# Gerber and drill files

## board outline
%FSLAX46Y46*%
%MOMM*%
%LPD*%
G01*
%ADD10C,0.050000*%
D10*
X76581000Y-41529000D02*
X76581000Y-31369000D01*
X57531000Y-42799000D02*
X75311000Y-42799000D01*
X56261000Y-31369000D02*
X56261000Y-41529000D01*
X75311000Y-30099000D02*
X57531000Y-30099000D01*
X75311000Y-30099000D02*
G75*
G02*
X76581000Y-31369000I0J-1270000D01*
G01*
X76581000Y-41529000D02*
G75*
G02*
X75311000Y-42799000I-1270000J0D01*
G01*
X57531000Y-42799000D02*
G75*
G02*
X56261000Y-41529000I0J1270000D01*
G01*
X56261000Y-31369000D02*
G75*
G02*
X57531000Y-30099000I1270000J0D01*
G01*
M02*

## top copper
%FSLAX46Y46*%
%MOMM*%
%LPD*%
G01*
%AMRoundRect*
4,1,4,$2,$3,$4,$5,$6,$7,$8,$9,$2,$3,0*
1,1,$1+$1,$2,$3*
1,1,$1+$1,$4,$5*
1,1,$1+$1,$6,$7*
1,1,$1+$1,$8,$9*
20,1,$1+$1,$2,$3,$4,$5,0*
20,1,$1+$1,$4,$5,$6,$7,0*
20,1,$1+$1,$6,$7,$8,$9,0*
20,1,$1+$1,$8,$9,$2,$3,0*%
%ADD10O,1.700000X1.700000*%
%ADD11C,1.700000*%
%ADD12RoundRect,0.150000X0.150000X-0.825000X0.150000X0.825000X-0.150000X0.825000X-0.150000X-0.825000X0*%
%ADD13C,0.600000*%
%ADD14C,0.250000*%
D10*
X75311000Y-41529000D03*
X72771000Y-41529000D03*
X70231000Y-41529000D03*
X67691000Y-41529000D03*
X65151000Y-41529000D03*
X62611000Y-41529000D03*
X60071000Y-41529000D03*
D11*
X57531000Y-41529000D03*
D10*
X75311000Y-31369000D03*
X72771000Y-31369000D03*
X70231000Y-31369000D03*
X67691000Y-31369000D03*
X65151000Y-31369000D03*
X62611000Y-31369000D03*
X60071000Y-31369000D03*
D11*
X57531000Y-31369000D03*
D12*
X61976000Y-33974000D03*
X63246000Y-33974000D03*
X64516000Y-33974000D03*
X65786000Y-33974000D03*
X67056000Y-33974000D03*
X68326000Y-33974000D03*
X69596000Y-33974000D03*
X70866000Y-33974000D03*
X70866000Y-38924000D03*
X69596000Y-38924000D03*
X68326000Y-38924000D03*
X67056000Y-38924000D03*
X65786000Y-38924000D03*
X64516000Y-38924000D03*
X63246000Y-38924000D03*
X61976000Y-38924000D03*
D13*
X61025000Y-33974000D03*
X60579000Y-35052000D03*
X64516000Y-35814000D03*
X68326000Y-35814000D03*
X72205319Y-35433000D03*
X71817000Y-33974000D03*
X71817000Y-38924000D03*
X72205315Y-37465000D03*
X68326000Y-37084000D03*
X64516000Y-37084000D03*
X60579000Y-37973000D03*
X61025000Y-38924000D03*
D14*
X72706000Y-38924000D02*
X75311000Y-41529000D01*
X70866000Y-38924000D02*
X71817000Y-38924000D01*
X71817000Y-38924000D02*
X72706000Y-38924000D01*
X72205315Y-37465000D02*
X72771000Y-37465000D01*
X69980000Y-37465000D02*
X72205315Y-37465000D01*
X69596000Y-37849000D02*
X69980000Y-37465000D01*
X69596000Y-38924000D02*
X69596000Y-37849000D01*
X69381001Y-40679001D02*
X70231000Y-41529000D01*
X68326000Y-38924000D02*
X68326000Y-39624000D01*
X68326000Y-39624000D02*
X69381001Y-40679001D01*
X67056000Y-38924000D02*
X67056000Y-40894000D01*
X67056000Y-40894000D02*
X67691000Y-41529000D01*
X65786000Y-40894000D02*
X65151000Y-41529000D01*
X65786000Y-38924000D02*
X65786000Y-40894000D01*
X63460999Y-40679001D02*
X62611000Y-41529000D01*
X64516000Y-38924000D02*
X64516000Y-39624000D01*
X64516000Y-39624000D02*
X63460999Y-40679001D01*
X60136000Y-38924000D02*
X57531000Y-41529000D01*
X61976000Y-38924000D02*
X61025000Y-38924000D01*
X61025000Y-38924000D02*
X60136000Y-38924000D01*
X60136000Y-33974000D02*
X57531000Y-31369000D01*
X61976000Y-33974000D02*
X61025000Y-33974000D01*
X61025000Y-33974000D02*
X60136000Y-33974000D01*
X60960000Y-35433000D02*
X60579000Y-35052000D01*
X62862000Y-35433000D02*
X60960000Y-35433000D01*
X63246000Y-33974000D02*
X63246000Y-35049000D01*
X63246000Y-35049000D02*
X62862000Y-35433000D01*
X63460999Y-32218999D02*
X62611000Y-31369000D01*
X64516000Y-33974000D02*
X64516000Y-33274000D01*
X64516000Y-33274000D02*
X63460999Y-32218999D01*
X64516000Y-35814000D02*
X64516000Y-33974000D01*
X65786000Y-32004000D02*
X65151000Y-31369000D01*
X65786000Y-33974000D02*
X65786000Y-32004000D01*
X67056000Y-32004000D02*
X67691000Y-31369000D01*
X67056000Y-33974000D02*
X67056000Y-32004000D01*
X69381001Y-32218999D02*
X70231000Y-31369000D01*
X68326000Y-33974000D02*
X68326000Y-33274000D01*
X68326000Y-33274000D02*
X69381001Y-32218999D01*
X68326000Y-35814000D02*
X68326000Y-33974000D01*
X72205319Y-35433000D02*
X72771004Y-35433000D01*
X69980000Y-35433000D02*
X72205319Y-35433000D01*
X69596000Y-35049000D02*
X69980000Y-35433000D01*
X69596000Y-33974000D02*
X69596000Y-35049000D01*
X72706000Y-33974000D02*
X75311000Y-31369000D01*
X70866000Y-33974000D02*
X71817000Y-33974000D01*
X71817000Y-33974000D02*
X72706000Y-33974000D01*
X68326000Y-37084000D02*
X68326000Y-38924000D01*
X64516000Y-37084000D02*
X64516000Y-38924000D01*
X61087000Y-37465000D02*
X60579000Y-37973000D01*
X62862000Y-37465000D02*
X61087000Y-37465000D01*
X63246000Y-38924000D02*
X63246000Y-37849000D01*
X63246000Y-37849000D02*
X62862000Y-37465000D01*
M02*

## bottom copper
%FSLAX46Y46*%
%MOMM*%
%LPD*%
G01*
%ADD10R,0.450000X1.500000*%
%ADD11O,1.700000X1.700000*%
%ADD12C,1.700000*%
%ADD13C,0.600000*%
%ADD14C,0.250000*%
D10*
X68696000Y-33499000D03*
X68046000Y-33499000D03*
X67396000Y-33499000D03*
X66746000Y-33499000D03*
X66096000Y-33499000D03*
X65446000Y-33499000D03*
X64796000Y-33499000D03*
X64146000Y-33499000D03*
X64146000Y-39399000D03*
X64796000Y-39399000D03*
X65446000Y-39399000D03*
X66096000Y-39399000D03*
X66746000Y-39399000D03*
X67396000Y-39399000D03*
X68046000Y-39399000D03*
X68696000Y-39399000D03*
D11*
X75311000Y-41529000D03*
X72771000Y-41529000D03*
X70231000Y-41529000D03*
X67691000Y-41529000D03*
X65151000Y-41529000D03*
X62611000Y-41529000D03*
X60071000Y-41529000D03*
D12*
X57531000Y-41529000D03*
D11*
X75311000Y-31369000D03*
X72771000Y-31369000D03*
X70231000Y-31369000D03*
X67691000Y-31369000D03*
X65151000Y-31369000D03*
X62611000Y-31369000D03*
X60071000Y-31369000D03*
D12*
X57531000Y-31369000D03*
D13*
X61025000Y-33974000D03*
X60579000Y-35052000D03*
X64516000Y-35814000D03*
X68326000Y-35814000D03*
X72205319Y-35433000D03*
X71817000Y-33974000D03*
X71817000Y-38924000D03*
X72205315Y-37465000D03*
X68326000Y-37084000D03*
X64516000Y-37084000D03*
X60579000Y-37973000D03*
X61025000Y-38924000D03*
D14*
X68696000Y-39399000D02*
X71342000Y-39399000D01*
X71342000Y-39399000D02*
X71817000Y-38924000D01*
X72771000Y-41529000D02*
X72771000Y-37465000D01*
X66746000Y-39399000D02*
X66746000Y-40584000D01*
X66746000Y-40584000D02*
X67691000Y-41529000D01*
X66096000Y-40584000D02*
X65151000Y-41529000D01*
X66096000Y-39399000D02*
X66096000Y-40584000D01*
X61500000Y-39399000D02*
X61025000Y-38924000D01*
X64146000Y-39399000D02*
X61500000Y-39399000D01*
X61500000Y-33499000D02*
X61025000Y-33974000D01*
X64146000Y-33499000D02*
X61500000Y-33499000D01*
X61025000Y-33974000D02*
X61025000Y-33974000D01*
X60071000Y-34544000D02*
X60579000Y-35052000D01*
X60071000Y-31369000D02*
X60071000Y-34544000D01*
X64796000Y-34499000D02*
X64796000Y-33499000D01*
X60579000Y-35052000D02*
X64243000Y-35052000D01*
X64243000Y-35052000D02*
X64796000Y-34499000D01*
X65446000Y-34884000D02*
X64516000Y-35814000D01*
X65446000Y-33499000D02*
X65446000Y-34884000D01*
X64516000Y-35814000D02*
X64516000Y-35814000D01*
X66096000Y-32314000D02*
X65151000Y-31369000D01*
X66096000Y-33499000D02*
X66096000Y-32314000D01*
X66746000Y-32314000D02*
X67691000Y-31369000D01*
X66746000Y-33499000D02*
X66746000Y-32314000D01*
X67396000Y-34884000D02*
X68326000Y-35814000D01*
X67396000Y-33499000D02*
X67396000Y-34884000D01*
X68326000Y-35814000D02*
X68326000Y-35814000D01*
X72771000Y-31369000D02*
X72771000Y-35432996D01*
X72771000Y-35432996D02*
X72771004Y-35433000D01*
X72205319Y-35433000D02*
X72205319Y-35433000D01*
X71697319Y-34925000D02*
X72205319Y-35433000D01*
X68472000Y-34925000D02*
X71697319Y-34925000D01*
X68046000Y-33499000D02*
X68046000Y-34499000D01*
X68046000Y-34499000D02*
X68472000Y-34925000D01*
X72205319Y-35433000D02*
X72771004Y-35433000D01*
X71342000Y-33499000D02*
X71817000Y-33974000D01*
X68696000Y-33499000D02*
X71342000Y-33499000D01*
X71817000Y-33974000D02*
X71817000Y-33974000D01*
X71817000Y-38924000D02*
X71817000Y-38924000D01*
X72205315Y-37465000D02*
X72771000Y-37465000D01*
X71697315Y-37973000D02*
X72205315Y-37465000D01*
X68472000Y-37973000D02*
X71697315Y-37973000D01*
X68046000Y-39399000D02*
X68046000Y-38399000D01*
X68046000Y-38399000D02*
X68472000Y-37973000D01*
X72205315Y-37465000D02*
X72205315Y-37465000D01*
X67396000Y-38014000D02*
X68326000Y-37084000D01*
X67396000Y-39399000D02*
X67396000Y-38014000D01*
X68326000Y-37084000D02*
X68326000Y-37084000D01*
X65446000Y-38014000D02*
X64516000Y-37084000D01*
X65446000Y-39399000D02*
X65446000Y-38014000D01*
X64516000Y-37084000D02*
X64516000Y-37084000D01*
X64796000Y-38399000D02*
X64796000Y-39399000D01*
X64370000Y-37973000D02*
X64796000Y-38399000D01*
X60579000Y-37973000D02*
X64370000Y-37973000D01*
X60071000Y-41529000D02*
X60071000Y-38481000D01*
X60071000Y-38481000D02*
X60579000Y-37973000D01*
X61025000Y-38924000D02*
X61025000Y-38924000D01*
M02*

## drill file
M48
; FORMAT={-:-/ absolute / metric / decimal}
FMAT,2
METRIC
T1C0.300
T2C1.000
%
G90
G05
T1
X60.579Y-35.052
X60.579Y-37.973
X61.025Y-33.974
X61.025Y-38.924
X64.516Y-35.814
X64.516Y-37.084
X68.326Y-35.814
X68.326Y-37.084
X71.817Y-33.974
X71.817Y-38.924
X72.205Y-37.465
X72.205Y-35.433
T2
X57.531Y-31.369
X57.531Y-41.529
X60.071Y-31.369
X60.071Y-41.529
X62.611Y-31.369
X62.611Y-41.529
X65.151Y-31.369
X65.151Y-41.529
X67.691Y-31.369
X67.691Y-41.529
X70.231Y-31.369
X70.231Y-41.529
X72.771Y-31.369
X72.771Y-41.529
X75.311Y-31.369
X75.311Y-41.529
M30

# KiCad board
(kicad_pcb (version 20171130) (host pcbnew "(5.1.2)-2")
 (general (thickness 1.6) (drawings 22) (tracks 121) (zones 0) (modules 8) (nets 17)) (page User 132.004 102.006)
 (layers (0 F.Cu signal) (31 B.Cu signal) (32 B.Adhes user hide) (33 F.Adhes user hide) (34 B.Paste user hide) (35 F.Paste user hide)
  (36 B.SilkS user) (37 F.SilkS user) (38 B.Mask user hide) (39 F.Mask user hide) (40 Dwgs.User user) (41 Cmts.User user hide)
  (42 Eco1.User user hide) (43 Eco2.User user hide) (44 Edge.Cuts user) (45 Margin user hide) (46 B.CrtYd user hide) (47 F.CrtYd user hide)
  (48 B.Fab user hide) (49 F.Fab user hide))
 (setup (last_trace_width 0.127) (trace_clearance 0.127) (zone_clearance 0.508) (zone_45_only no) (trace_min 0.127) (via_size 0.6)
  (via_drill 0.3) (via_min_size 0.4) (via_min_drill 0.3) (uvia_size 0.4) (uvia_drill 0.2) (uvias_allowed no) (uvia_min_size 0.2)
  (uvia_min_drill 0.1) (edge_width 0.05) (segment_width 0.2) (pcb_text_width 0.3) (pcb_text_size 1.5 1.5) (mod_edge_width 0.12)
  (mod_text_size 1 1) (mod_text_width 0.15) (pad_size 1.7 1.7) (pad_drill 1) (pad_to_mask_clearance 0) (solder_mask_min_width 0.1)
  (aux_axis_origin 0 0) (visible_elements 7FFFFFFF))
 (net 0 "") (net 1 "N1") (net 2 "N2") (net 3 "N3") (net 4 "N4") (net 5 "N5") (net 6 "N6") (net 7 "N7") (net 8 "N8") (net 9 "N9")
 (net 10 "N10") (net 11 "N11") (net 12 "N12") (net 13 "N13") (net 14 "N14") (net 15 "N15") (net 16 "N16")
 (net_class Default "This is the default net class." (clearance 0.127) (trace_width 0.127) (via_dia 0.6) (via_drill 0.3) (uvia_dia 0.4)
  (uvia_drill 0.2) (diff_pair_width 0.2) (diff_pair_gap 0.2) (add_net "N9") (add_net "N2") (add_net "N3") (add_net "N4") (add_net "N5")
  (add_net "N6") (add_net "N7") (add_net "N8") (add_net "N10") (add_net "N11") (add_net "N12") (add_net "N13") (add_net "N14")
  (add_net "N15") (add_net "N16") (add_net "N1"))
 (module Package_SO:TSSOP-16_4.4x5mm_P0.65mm (layer B.Cu) (at 66.421 36.449 90)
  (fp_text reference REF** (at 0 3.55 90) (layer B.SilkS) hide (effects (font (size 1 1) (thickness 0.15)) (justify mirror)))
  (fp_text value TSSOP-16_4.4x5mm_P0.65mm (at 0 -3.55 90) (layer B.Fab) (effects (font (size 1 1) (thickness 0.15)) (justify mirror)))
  (pad 16 smd rect (at 2.95 2.275 90) (size 1.5 0.45) (layers B.Cu B.Paste B.Mask) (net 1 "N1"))
  (pad 15 smd rect (at 2.95 1.625 90) (size 1.5 0.45) (layers B.Cu B.Paste B.Mask) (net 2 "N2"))
  (pad 14 smd rect (at 2.95 0.975 90) (size 1.5 0.45) (layers B.Cu B.Paste B.Mask) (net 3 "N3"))
  (pad 13 smd rect (at 2.95 0.325 90) (size 1.5 0.45) (layers B.Cu B.Paste B.Mask) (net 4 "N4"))
  (pad 12 smd rect (at 2.95 -0.325 90) (size 1.5 0.45) (layers B.Cu B.Paste B.Mask) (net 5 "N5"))
  (pad 11 smd rect (at 2.95 -0.975 90) (size 1.5 0.45) (layers B.Cu B.Paste B.Mask) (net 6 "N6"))
  (pad 10 smd rect (at 2.95 -1.625 90) (size 1.5 0.45) (layers B.Cu B.Paste B.Mask) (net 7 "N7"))
  (pad 9 smd rect (at 2.95 -2.275 90) (size 1.5 0.45) (layers B.Cu B.Paste B.Mask) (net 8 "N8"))
  (pad 8 smd rect (at -2.95 -2.275 90) (size 1.5 0.45) (layers B.Cu B.Paste B.Mask) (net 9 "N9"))
  (pad 7 smd rect (at -2.95 -1.625 90) (size 1.5 0.45) (layers B.Cu B.Paste B.Mask) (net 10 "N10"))
  (pad 6 smd rect (at -2.95 -0.975 90) (size 1.5 0.45) (layers B.Cu B.Paste B.Mask) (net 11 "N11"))
  (pad 5 smd rect (at -2.95 -0.325 90) (size 1.5 0.45) (layers B.Cu B.Paste B.Mask) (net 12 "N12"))
  (pad 4 smd rect (at -2.95 0.325 90) (size 1.5 0.45) (layers B.Cu B.Paste B.Mask) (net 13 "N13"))
  (pad 3 smd rect (at -2.95 0.975 90) (size 1.5 0.45) (layers B.Cu B.Paste B.Mask) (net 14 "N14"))
  (pad 2 smd rect (at -2.95 1.625 90) (size 1.5 0.45) (layers B.Cu B.Paste B.Mask) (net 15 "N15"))
  (pad 1 smd rect (at -2.95 2.275 90) (size 1.5 0.45) (layers B.Cu B.Paste B.Mask) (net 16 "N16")))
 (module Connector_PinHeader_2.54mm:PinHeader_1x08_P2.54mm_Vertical (layer F.Cu) (at 57.531 41.529 90)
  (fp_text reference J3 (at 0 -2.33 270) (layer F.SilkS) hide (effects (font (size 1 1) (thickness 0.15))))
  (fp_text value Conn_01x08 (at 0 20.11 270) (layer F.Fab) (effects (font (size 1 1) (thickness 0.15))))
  (pad 8 thru_hole oval (at 0 17.78 90) (size 1.7 1.7) (drill 1) (layers *.Cu *.Mask) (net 16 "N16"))
  (pad 7 thru_hole oval (at 0 15.24 90) (size 1.7 1.7) (drill 1) (layers *.Cu *.Mask) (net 15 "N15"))
  (pad 6 thru_hole oval (at 0 12.7 90) (size 1.7 1.7) (drill 1) (layers *.Cu *.Mask) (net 14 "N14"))
  (pad 5 thru_hole oval (at 0 10.16 90) (size 1.7 1.7) (drill 1) (layers *.Cu *.Mask) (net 13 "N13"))
  (pad 4 thru_hole oval (at 0 7.62 90) (size 1.7 1.7) (drill 1) (layers *.Cu *.Mask) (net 12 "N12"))
  (pad 3 thru_hole oval (at 0 5.08 90) (size 1.7 1.7) (drill 1) (layers *.Cu *.Mask) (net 11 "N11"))
  (pad 2 thru_hole oval (at 0 2.54 90) (size 1.7 1.7) (drill 1) (layers *.Cu *.Mask) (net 10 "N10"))
  (pad 1 thru_hole circle (at 0 0 90) (size 1.7 1.7) (drill 1) (layers *.Cu *.Mask) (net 9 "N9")))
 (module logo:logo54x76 (layer F.Cu) (at 58.801 36.703)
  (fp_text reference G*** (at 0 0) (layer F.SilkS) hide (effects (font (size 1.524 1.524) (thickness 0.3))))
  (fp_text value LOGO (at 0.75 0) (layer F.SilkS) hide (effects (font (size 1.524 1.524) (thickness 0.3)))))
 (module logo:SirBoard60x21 (layer F.Cu) (at 66.421 36.449)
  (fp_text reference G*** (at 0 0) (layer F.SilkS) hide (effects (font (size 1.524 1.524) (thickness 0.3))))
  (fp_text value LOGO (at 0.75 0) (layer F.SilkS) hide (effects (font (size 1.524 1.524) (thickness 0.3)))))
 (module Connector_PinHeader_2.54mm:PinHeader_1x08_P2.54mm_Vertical (layer F.Cu) (at 57.531 31.369 90)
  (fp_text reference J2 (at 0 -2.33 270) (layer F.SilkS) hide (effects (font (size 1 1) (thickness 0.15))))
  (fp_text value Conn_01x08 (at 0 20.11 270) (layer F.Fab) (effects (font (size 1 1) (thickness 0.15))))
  (pad 8 thru_hole oval (at 0 17.78 90) (size 1.7 1.7) (drill 1) (layers *.Cu *.Mask) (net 1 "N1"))
  (pad 7 thru_hole oval (at 0 15.24 90) (size 1.7 1.7) (drill 1) (layers *.Cu *.Mask) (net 2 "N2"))
  (pad 6 thru_hole oval (at 0 12.7 90) (size 1.7 1.7) (drill 1) (layers *.Cu *.Mask) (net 3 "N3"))
  (pad 5 thru_hole oval (at 0 10.16 90) (size 1.7 1.7) (drill 1) (layers *.Cu *.Mask) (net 4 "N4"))
  (pad 4 thru_hole oval (at 0 7.62 90) (size 1.7 1.7) (drill 1) (layers *.Cu *.Mask) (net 5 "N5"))
  (pad 3 thru_hole oval (at 0 5.08 90) (size 1.7 1.7) (drill 1) (layers *.Cu *.Mask) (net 6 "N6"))
  (pad 2 thru_hole oval (at 0 2.54 90) (size 1.7 1.7) (drill 1) (layers *.Cu *.Mask) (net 7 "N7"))
  (pad 1 thru_hole circle (at 0 0 90) (size 1.7 1.7) (drill 1) (layers *.Cu *.Mask) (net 8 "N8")))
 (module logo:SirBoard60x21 (layer B.Cu) (at 59.182 36.449 90)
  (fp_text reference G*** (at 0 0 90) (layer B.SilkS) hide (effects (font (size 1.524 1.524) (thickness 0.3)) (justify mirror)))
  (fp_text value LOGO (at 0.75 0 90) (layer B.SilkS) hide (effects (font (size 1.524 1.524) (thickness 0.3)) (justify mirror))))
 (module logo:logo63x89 (layer B.Cu) (at 73.025 36.576 90)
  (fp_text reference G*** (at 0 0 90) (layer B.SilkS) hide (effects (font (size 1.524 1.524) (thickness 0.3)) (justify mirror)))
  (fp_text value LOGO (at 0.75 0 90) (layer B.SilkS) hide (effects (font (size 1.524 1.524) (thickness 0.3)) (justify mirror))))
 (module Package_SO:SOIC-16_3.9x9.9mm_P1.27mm (layer F.Cu) (at 66.421 36.449 90)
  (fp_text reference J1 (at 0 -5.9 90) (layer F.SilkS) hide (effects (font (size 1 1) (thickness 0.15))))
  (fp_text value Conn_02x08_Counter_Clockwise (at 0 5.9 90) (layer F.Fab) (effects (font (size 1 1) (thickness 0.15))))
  (pad 16 smd roundrect (at 2.475 -4.445 90) (size 1.95 0.6) (layers F.Cu F.Paste F.Mask) (roundrect_rratio 0.25) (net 8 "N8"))
  (pad 15 smd roundrect (at 2.475 -3.175 90) (size 1.95 0.6) (layers F.Cu F.Paste F.Mask) (roundrect_rratio 0.25) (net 7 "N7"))
  (pad 14 smd roundrect (at 2.475 -1.905 90) (size 1.95 0.6) (layers F.Cu F.Paste F.Mask) (roundrect_rratio 0.25) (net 6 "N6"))
  (pad 13 smd roundrect (at 2.475 -0.635 90) (size 1.95 0.6) (layers F.Cu F.Paste F.Mask) (roundrect_rratio 0.25) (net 5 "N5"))
  (pad 12 smd roundrect (at 2.475 0.635 90) (size 1.95 0.6) (layers F.Cu F.Paste F.Mask) (roundrect_rratio 0.25) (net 4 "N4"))
  (pad 11 smd roundrect (at 2.475 1.905 90) (size 1.95 0.6) (layers F.Cu F.Paste F.Mask) (roundrect_rratio 0.25) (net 3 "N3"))
  (pad 10 smd roundrect (at 2.475 3.175 90) (size 1.95 0.6) (layers F.Cu F.Paste F.Mask) (roundrect_rratio 0.25) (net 2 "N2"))
  (pad 9 smd roundrect (at 2.475 4.445 90) (size 1.95 0.6) (layers F.Cu F.Paste F.Mask) (roundrect_rratio 0.25) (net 1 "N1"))
  (pad 8 smd roundrect (at -2.475 4.445 90) (size 1.95 0.6) (layers F.Cu F.Paste F.Mask) (roundrect_rratio 0.25) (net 16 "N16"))
  (pad 7 smd roundrect (at -2.475 3.175 90) (size 1.95 0.6) (layers F.Cu F.Paste F.Mask) (roundrect_rratio 0.25) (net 15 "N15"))
  (pad 6 smd roundrect (at -2.475 1.905 90) (size 1.95 0.6) (layers F.Cu F.Paste F.Mask) (roundrect_rratio 0.25) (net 14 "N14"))
  (pad 5 smd roundrect (at -2.475 0.635 90) (size 1.95 0.6) (layers F.Cu F.Paste F.Mask) (roundrect_rratio 0.25) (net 13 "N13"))
  (pad 4 smd roundrect (at -2.475 -0.635 90) (size 1.95 0.6) (layers F.Cu F.Paste F.Mask) (roundrect_rratio 0.25) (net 12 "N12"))
  (pad 3 smd roundrect (at -2.475 -1.905 90) (size 1.95 0.6) (layers F.Cu F.Paste F.Mask) (roundrect_rratio 0.25) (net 11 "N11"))
  (pad 2 smd roundrect (at -2.475 -3.175 90) (size 1.95 0.6) (layers F.Cu F.Paste F.Mask) (roundrect_rratio 0.25) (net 10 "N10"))
  (pad 1 smd roundrect (at -2.475 -4.445 90) (size 1.95 0.6) (layers F.Cu F.Paste F.Mask) (roundrect_rratio 0.25) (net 9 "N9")))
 (gr_line (start 76.581 41.529) (end 76.581 31.369) (layer Edge.Cuts) (width 0.05))
 (gr_line (start 57.531 42.799) (end 75.311 42.799) (layer Edge.Cuts) (width 0.05))
 (gr_line (start 56.261 31.369) (end 56.261 41.529) (layer Edge.Cuts) (width 0.05))
 (gr_line (start 75.311 30.099) (end 57.531 30.099) (layer Edge.Cuts) (width 0.05))
 (gr_arc (start 75.311 31.369) (end 76.581 31.369) (angle -90) (layer Edge.Cuts) (width 0.05))
 (gr_arc (start 75.311 41.529) (end 75.311 42.799) (angle -90) (layer Edge.Cuts) (width 0.05))
 (gr_arc (start 57.531 41.529) (end 56.261 41.529) (angle -90) (layer Edge.Cuts) (width 0.05))
 (gr_arc (start 57.531 31.369) (end 57.531 30.099) (angle -90) (layer Edge.Cuts) (width 0.05))
 (segment (start 72.706 38.924) (end 75.311 41.529) (width 0.25) (layer F.Cu) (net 16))
 (segment (start 68.696 39.399) (end 71.342 39.399) (width 0.25) (layer B.Cu) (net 16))
 (segment (start 71.342 39.399) (end 71.817 38.924) (width 0.25) (layer B.Cu) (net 16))
 (segment (start 70.866 38.924) (end 71.817 38.924) (width 0.25) (layer F.Cu) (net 16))
 (segment (start 71.817 38.924) (end 72.706 38.924) (width 0.25) (layer F.Cu) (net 16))
 (segment (start 72.771 41.529) (end 72.771 37.465) (width 0.25) (layer B.Cu) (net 15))
 (segment (start 72.205315 37.465) (end 72.771 37.465) (width 0.25) (layer F.Cu) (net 15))
 (segment (start 69.98 37.465) (end 72.205315 37.465) (width 0.25) (layer F.Cu) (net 15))
 (segment (start 69.596 37.849) (end 69.98 37.465) (width 0.25) (layer F.Cu) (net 15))
 (segment (start 69.596 38.924) (end 69.596 37.849) (width 0.25) (layer F.Cu) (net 15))
 (segment (start 69.381001 40.679001) (end 70.231 41.529) (width 0.25) (layer F.Cu) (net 14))
 (segment (start 68.326 38.924) (end 68.326 39.624) (width 0.25) (layer F.Cu) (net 14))
 (segment (start 68.326 39.624) (end 69.381001 40.679001) (width 0.25) (layer F.Cu) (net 14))
 (segment (start 66.746 39.399) (end 66.746 40.584) (width 0.25) (layer B.Cu) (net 13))
 (segment (start 66.746 40.584) (end 67.691 41.529) (width 0.25) (layer B.Cu) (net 13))
 (segment (start 67.056 38.924) (end 67.056 40.894) (width 0.25) (layer F.Cu) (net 13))
 (segment (start 67.056 40.894) (end 67.691 41.529) (width 0.25) (layer F.Cu) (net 13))
 (segment (start 65.786 40.894) (end 65.151 41.529) (width 0.25) (layer F.Cu) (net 12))
 (segment (start 65.786 38.924) (end 65.786 40.894) (width 0.25) (layer F.Cu) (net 12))
 (segment (start 66.096 40.584) (end 65.151 41.529) (width 0.25) (layer B.Cu) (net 12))
 (segment (start 66.096 39.399) (end 66.096 40.584) (width 0.25) (layer B.Cu) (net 12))
 (segment (start 63.460999 40.679001) (end 62.611 41.529) (width 0.25) (layer F.Cu) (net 11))
 (segment (start 64.516 38.924) (end 64.516 39.624) (width 0.25) (layer F.Cu) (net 11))
 (segment (start 64.516 39.624) (end 63.460999 40.679001) (width 0.25) (layer F.Cu) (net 11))
 (segment (start 60.136 38.924) (end 57.531 41.529) (width 0.25) (layer F.Cu) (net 9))
 (segment (start 61.5 39.399) (end 61.025 38.924) (width 0.25) (layer B.Cu) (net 9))
 (segment (start 61.976 38.924) (end 61.025 38.924) (width 0.25) (layer F.Cu) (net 9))
 (segment (start 61.025 38.924) (end 60.136 38.924) (width 0.25) (layer F.Cu) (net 9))
 (segment (start 64.146 39.399) (end 61.5 39.399) (width 0.25) (layer B.Cu) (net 9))
 (segment (start 60.136 33.974) (end 57.531 31.369) (width 0.25) (layer F.Cu) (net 8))
 (segment (start 61.5 33.499) (end 61.025 33.974) (width 0.25) (layer B.Cu) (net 8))
 (segment (start 64.146 33.499) (end 61.5 33.499) (width 0.25) (layer B.Cu) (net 8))
 (segment (start 61.976 33.974) (end 61.025 33.974) (width 0.25) (layer F.Cu) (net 8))
 (segment (start 61.025 33.974) (end 60.136 33.974) (width 0.25) (layer F.Cu) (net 8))
 (segment (start 61.025 33.974) (end 61.025 33.974) (width 0.25) (layer B.Cu) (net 8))
 (via (at 61.025 33.974) (size 0.6) (drill 0.3) (layers F.Cu B.Cu) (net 8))
 (via (at 60.579 35.052) (size 0.6) (drill 0.3) (layers F.Cu B.Cu) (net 7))
 (segment (start 60.071 34.544) (end 60.579 35.052) (width 0.25) (layer B.Cu) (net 7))
 (segment (start 60.071 31.369) (end 60.071 34.544) (width 0.25) (layer B.Cu) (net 7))
 (segment (start 64.796 34.499) (end 64.796 33.499) (width 0.25) (layer B.Cu) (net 7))
 (segment (start 60.579 35.052) (end 64.243 35.052) (width 0.25) (layer B.Cu) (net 7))
 (segment (start 64.243 35.052) (end 64.796 34.499) (width 0.25) (layer B.Cu) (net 7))
 (segment (start 60.96 35.433) (end 60.579 35.052) (width 0.25) (layer F.Cu) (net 7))
 (segment (start 62.862 35.433) (end 60.96 35.433) (width 0.25) (layer F.Cu) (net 7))
 (segment (start 63.246 33.974) (end 63.246 35.049) (width 0.25) (layer F.Cu) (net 7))
 (segment (start 63.246 35.049) (end 62.862 35.433) (width 0.25) (layer F.Cu) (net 7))
 (segment (start 63.460999 32.218999) (end 62.611 31.369) (width 0.25) (layer F.Cu) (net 6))
 (segment (start 64.516 33.974) (end 64.516 33.274) (width 0.25) (layer F.Cu) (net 6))
 (segment (start 64.516 33.274) (end 63.460999 32.218999) (width 0.25) (layer F.Cu) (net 6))
 (segment (start 65.446 34.884) (end 64.516 35.814) (width 0.25) (layer B.Cu) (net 6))
 (segment (start 65.446 33.499) (end 65.446 34.884) (width 0.25) (layer B.Cu) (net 6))
 (segment (start 64.516 35.814) (end 64.516 33.974) (width 0.25) (layer F.Cu) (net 6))
 (segment (start 64.516 35.814) (end 64.516 35.814) (width 0.25) (layer B.Cu) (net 6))
 (via (at 64.516 35.814) (size 0.6) (drill 0.3) (layers F.Cu B.Cu) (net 6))
 (segment (start 65.786 32.004) (end 65.151 31.369) (width 0.25) (layer F.Cu) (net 5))
 (segment (start 65.786 33.974) (end 65.786 32.004) (width 0.25) (layer F.Cu) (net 5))
 (segment (start 66.096 32.314) (end 65.151 31.369) (width 0.25) (layer B.Cu) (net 5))
 (segment (start 66.096 33.499) (end 66.096 32.314) (width 0.25) (layer B.Cu) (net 5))
 (segment (start 67.056 32.004) (end 67.691 31.369) (width 0.25) (layer F.Cu) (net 4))
 (segment (start 67.056 33.974) (end 67.056 32.004) (width 0.25) (layer F.Cu) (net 4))
 (segment (start 66.746 32.314) (end 67.691 31.369) (width 0.25) (layer B.Cu) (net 4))
 (segment (start 66.746 33.499) (end 66.746 32.314) (width 0.25) (layer B.Cu) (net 4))
 (segment (start 69.381001 32.218999) (end 70.231 31.369) (width 0.25) (layer F.Cu) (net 3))
 (segment (start 68.326 33.974) (end 68.326 33.274) (width 0.25) (layer F.Cu) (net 3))
 (segment (start 68.326 33.274) (end 69.381001 32.218999) (width 0.25) (layer F.Cu) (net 3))
 (segment (start 67.396 34.884) (end 68.326 35.814) (width 0.25) (layer B.Cu) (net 3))
 (segment (start 67.396 33.499) (end 67.396 34.884) (width 0.25) (layer B.Cu) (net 3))
 (segment (start 68.326 35.814) (end 68.326 33.974) (width 0.25) (layer F.Cu) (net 3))
 (segment (start 68.326 35.814) (end 68.326 35.814) (width 0.25) (layer B.Cu) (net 3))
 (via (at 68.326 35.814) (size 0.6) (drill 0.3) (layers F.Cu B.Cu) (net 3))
 (segment (start 72.205319 35.433) (end 72.771004 35.433) (width 0.25) (layer F.Cu) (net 2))
 (segment (start 69.98 35.433) (end 72.205319 35.433) (width 0.25) (layer F.Cu) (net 2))
 (segment (start 69.596 35.049) (end 69.98 35.433) (width 0.25) (layer F.Cu) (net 2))
 (segment (start 69.596 33.974) (end 69.596 35.049) (width 0.25) (layer F.Cu) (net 2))
 (segment (start 72.771 31.369) (end 72.771 35.432996) (width 0.25) (layer B.Cu) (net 2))
 (segment (start 72.771 35.432996) (end 72.771004 35.433) (width 0.25) (layer B.Cu) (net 2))
 (segment (start 72.205319 35.433) (end 72.205319 35.433) (width 0.25) (layer B.Cu) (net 2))
 (segment (start 71.697319 34.925) (end 72.205319 35.433) (width 0.25) (layer B.Cu) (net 2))
 (segment (start 68.472 34.925) (end 71.697319 34.925) (width 0.25) (layer B.Cu) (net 2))
 (segment (start 68.046 33.499) (end 68.046 34.499) (width 0.25) (layer B.Cu) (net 2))
 (segment (start 68.046 34.499) (end 68.472 34.925) (width 0.25) (layer B.Cu) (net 2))
 (segment (start 72.205319 35.433) (end 72.771004 35.433) (width 0.25) (layer B.Cu) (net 2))
 (via (at 72.205319 35.433) (size 0.6) (drill 0.3) (layers F.Cu B.Cu) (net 2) (status 1000000))
 (segment (start 72.706 33.974) (end 75.311 31.369) (width 0.25) (layer F.Cu) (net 1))
 (segment (start 71.342 33.499) (end 71.817 33.974) (width 0.25) (layer B.Cu) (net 1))
 (segment (start 68.696 33.499) (end 71.342 33.499) (width 0.25) (layer B.Cu) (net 1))
 (segment (start 70.866 33.974) (end 71.817 33.974) (width 0.25) (layer F.Cu) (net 1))
 (segment (start 71.817 33.974) (end 72.706 33.974) (width 0.25) (layer F.Cu) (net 1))
 (segment (start 71.817 33.974) (end 71.817 33.974) (width 0.25) (layer B.Cu) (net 1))
 (via (at 71.817 33.974) (size 0.6) (drill 0.3) (layers F.Cu B.Cu) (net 1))
 (segment (start 71.817 38.924) (end 71.817 38.924) (width 0.25) (layer B.Cu) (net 16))
 (via (at 71.817 38.924) (size 0.6) (drill 0.3) (layers F.Cu B.Cu) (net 16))
 (segment (start 72.205315 37.465) (end 72.771 37.465) (width 0.25) (layer B.Cu) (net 15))
 (segment (start 71.697315 37.973) (end 72.205315 37.465) (width 0.25) (layer B.Cu) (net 15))
 (segment (start 68.472 37.973) (end 71.697315 37.973) (width 0.25) (layer B.Cu) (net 15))
 (segment (start 68.046 39.399) (end 68.046 38.399) (width 0.25) (layer B.Cu) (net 15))
 (segment (start 68.046 38.399) (end 68.472 37.973) (width 0.25) (layer B.Cu) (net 15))
 (segment (start 72.205315 37.465) (end 72.205315 37.465) (width 0.25) (layer B.Cu) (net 15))
 (via (at 72.205315 37.465) (size 0.6) (drill 0.3) (layers F.Cu B.Cu) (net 15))
 (segment (start 67.396 38.014) (end 68.326 37.084) (width 0.25) (layer B.Cu) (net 14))
 (segment (start 67.396 39.399) (end 67.396 38.014) (width 0.25) (layer B.Cu) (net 14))
 (segment (start 68.326 37.084) (end 68.326 38.924) (width 0.25) (layer F.Cu) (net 14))
 (segment (start 68.326 37.084) (end 68.326 37.084) (width 0.25) (layer B.Cu) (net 14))
 (via (at 68.326 37.084) (size 0.6) (drill 0.3) (layers F.Cu B.Cu) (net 14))
 (segment (start 64.516 37.084) (end 64.516 38.924) (width 0.25) (layer F.Cu) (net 11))
 (segment (start 65.446 38.014) (end 64.516 37.084) (width 0.25) (layer B.Cu) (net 11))
 (segment (start 65.446 39.399) (end 65.446 38.014) (width 0.25) (layer B.Cu) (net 11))
 (segment (start 64.516 37.084) (end 64.516 37.084) (width 0.25) (layer B.Cu) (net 11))
 (via (at 64.516 37.084) (size 0.6) (drill 0.3) (layers F.Cu B.Cu) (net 11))
 (via (at 60.579 37.973) (size 0.6) (drill 0.3) (layers F.Cu B.Cu) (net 10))
 (segment (start 64.796 38.399) (end 64.796 39.399) (width 0.25) (layer B.Cu) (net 10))
 (segment (start 64.37 37.973) (end 64.796 38.399) (width 0.25) (layer B.Cu) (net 10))
 (segment (start 60.579 37.973) (end 64.37 37.973) (width 0.25) (layer B.Cu) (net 10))
 (segment (start 60.071 41.529) (end 60.071 38.481) (width 0.25) (layer B.Cu) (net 10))
 (segment (start 60.071 38.481) (end 60.579 37.973) (width 0.25) (layer B.Cu) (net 10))
 (segment (start 61.087 37.465) (end 60.579 37.973) (width 0.25) (layer F.Cu) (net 10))
 (segment (start 62.862 37.465) (end 61.087 37.465) (width 0.25) (layer F.Cu) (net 10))
 (segment (start 63.246 38.924) (end 63.246 37.849) (width 0.25) (layer F.Cu) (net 10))
 (segment (start 63.246 37.849) (end 62.862 37.465) (width 0.25) (layer F.Cu) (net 10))
 (segment (start 61.025 38.924) (end 61.025 38.924) (width 0.25) (layer B.Cu) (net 9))
 (via (at 61.025 38.924) (size 0.6) (drill 0.3) (layers F.Cu B.Cu) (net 9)))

